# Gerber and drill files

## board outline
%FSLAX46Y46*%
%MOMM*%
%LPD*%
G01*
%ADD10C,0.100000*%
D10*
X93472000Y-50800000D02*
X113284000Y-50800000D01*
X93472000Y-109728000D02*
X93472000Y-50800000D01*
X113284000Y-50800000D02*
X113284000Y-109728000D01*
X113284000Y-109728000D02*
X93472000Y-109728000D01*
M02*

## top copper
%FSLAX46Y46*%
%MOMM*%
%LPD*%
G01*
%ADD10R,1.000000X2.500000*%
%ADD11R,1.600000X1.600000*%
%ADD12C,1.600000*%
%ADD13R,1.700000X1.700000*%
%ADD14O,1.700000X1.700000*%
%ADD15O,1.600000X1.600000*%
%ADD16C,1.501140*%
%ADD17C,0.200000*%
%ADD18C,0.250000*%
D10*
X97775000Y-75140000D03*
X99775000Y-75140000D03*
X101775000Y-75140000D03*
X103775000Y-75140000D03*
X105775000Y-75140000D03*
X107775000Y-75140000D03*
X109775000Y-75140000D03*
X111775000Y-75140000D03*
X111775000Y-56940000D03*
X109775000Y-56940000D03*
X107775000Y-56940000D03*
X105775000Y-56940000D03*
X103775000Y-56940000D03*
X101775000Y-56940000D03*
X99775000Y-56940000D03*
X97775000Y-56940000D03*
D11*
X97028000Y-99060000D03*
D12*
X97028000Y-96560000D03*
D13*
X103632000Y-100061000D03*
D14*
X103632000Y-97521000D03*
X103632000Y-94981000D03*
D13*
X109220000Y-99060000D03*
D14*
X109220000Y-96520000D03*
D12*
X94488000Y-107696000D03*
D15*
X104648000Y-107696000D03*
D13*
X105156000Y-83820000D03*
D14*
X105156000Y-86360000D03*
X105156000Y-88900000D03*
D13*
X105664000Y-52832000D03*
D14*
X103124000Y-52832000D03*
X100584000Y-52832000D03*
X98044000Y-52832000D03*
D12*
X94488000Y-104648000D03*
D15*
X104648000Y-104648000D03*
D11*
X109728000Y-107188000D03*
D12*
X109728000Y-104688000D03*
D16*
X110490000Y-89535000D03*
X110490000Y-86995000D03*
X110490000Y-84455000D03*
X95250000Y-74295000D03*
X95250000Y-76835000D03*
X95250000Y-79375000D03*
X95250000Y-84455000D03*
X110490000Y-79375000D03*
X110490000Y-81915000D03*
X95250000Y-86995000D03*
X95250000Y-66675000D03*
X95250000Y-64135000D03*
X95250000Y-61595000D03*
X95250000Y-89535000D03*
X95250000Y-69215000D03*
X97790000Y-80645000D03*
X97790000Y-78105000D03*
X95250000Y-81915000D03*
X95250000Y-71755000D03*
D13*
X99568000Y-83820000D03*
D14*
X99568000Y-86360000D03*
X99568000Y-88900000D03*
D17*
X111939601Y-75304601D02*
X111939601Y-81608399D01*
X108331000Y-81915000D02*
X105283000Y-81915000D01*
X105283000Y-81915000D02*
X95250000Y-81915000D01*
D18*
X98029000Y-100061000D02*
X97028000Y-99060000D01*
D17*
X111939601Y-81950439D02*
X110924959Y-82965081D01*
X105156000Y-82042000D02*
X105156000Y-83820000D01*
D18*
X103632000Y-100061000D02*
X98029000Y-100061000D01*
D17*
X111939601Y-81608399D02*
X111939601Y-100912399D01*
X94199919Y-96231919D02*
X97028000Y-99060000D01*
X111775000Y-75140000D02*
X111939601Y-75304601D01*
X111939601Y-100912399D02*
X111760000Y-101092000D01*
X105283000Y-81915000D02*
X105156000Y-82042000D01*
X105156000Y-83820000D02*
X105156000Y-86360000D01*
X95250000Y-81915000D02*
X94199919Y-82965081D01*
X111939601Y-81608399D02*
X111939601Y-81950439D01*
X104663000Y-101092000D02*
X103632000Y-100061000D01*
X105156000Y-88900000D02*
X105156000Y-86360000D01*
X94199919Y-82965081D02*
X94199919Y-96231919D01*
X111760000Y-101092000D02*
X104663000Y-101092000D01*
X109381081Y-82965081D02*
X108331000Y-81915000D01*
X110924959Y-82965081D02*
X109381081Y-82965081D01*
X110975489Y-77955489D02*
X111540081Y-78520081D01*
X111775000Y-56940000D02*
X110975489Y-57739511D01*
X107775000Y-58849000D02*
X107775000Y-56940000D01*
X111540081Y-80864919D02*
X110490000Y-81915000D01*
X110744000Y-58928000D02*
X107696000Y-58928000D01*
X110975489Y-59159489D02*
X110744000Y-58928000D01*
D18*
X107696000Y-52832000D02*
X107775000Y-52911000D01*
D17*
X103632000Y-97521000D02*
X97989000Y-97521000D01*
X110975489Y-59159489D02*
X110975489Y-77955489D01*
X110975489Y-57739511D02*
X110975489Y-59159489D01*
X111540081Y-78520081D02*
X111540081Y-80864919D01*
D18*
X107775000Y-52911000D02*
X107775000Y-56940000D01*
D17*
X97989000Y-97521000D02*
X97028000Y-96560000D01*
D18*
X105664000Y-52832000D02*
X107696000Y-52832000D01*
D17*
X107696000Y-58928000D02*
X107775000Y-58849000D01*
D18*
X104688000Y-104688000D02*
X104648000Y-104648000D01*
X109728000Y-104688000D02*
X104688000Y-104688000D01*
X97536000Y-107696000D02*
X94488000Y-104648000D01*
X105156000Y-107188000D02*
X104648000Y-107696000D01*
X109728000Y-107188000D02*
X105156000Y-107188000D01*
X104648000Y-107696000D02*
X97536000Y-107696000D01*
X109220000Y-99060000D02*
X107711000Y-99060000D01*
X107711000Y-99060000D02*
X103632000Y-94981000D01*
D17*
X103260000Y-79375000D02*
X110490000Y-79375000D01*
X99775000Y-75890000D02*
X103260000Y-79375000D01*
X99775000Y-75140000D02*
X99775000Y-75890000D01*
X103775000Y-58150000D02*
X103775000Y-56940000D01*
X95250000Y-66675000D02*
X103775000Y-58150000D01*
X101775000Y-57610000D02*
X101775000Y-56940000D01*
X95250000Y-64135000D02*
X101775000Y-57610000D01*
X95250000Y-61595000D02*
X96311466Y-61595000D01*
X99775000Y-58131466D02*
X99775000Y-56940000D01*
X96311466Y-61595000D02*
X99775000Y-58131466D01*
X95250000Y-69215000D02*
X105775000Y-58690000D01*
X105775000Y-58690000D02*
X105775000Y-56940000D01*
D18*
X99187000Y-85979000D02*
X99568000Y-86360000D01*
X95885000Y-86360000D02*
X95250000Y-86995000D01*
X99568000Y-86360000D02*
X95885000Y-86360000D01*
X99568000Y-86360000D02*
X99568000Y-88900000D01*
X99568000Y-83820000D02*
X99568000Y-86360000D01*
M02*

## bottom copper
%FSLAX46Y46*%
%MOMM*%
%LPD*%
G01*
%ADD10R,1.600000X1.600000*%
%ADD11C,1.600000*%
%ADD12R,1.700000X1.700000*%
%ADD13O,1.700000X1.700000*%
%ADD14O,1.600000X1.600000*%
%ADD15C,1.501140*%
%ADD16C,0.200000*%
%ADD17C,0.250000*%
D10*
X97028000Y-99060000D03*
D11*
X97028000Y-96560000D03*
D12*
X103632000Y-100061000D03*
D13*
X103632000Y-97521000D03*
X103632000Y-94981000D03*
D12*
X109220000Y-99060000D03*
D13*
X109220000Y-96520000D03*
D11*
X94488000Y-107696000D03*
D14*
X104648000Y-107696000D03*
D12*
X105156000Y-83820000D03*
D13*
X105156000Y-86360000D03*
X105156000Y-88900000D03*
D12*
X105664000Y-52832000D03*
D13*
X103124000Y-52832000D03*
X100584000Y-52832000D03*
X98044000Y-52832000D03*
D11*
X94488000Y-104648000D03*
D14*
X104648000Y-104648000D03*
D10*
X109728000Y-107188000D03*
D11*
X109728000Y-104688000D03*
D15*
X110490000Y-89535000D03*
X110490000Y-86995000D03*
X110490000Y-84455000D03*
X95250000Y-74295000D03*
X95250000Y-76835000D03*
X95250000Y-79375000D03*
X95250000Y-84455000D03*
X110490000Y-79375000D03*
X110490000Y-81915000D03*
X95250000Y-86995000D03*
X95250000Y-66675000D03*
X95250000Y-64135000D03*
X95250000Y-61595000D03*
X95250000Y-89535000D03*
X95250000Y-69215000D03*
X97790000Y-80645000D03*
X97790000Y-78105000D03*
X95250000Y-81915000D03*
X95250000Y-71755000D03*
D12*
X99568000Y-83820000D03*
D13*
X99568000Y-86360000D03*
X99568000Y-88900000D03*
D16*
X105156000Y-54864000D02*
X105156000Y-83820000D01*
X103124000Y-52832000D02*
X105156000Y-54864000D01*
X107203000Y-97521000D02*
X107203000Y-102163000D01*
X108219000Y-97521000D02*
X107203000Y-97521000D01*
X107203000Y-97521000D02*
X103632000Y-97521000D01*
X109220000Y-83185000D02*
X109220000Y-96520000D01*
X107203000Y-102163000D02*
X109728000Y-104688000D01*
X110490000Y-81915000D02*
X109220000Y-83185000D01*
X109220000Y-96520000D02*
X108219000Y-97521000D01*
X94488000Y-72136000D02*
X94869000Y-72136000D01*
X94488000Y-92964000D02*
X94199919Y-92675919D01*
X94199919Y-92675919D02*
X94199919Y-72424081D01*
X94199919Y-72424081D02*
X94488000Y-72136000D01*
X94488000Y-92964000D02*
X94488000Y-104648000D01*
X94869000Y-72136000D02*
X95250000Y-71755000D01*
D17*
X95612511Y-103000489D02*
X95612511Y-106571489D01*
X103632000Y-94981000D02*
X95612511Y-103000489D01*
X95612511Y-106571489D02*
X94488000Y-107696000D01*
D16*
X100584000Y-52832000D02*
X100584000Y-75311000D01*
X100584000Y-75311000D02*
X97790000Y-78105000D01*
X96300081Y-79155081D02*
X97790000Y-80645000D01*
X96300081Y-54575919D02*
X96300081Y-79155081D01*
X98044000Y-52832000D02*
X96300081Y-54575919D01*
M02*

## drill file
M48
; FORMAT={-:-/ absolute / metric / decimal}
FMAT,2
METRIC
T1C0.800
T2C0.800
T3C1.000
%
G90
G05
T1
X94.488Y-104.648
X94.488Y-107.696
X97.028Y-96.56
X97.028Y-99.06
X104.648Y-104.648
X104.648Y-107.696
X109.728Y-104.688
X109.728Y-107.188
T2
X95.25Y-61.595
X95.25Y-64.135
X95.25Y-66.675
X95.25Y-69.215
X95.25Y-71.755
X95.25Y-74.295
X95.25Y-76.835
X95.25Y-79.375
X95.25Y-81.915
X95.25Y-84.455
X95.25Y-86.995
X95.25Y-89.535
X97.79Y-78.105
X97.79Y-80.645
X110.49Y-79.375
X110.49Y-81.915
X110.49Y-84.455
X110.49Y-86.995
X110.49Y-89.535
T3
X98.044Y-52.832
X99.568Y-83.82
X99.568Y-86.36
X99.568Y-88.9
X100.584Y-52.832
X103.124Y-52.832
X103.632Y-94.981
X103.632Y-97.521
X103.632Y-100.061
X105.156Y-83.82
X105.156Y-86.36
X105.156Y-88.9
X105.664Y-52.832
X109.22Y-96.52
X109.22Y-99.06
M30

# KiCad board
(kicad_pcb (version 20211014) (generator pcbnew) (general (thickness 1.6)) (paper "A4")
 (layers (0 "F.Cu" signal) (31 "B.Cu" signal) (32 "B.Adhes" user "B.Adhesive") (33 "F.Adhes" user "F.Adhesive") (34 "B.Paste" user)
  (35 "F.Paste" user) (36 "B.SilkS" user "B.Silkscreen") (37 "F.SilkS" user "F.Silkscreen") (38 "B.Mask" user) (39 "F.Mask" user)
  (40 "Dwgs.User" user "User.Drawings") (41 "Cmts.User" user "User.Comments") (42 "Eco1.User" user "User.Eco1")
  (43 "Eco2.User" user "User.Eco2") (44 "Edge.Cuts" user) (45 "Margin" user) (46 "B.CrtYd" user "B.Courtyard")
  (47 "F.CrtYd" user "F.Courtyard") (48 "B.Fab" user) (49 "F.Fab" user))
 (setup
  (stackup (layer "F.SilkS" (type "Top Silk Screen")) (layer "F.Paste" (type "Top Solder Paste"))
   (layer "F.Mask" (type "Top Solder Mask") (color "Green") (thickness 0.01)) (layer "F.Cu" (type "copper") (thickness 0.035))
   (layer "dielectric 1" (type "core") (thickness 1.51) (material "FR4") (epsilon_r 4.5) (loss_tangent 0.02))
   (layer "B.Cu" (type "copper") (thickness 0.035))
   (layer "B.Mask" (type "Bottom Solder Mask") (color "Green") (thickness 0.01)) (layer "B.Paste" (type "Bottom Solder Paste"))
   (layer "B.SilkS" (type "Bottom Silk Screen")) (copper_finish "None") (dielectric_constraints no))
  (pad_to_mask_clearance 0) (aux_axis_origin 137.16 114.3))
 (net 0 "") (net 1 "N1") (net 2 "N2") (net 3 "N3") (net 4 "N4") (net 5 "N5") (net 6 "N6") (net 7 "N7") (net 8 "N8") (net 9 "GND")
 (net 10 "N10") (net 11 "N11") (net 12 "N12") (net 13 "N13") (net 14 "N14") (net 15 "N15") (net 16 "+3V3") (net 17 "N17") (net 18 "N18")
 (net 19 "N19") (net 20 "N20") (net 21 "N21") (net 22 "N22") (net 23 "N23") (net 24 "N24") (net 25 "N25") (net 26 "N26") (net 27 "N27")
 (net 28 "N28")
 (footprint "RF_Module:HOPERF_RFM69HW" (layer "F.Cu") (at 104.775 66.04 90)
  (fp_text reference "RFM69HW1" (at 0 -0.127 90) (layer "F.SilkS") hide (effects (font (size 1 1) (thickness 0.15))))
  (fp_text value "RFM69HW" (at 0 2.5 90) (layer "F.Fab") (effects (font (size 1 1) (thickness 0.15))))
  (pad "1" smd rect (at -9.1 -7 90) (size 2.5 1) (layers "F.Cu" "F.Paste" "F.Mask") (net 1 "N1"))
  (pad "2" smd rect (at -9.1 -5 90) (size 2.5 1) (layers "F.Cu" "F.Paste" "F.Mask") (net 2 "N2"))
  (pad "3" smd rect (at -9.1 -3 90) (size 2.5 1) (layers "F.Cu" "F.Paste" "F.Mask") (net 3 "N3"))
  (pad "4" smd rect (at -9.1 -1 90) (size 2.5 1) (layers "F.Cu" "F.Paste" "F.Mask") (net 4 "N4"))
  (pad "5" smd rect (at -9.1 1 90) (size 2.5 1) (layers "F.Cu" "F.Paste" "F.Mask") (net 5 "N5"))
  (pad "6" smd rect (at -9.1 3 90) (size 2.5 1) (layers "F.Cu" "F.Paste" "F.Mask") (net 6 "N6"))
  (pad "7" smd rect (at -9.1 5 90) (size 2.5 1) (layers "F.Cu" "F.Paste" "F.Mask") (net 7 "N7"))
  (pad "8" smd rect (at -9.1 7 90) (size 2.5 1) (layers "F.Cu" "F.Paste" "F.Mask") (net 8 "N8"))
  (pad "9" smd rect (at 9.1 7 90) (size 2.5 1) (layers "F.Cu" "F.Paste" "F.Mask") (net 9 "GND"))
  (pad "10" smd rect (at 9.1 5 90) (size 2.5 1) (layers "F.Cu" "F.Paste" "F.Mask") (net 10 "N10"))
  (pad "11" smd rect (at 9.1 3 90) (size 2.5 1) (layers "F.Cu" "F.Paste" "F.Mask") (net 9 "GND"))
  (pad "12" smd rect (at 9.1 1 90) (size 2.5 1) (layers "F.Cu" "F.Paste" "F.Mask") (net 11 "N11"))
  (pad "13" smd rect (at 9.1 -1 90) (size 2.5 1) (layers "F.Cu" "F.Paste" "F.Mask") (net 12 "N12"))
  (pad "14" smd rect (at 9.1 -3 90) (size 2.5 1) (layers "F.Cu" "F.Paste" "F.Mask") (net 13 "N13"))
  (pad "15" smd rect (at 9.1 -5 90) (size 2.5 1) (layers "F.Cu" "F.Paste" "F.Mask") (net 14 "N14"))
  (pad "16" smd rect (at 9.1 -7 90) (size 2.5 1) (layers "F.Cu" "F.Paste" "F.Mask") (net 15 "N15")))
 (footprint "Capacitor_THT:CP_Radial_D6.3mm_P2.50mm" (layer "F.Cu") (at 97.028 99.06 90)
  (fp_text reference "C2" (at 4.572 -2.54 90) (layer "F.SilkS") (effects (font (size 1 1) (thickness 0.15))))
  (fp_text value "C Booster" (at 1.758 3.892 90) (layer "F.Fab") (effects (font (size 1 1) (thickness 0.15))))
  (pad "1" thru_hole rect (at 0 0 90) (size 1.6 1.6) (drill 0.8) (layers *.Cu *.Mask) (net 8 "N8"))
  (pad "2" thru_hole circle (at 2.5 0 90) (size 1.6 1.6) (drill 0.8) (layers *.Cu *.Mask) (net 9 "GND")))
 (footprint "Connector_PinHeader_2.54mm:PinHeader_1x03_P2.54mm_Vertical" (layer "F.Cu") (at 103.632 100.061 180)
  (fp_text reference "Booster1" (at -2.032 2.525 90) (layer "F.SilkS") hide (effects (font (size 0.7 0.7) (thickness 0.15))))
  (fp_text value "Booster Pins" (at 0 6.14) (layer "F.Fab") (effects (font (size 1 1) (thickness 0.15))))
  (pad "1" thru_hole rect (at 0 0 180) (size 1.7 1.7) (drill 1) (layers *.Cu *.Mask) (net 8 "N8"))
  (pad "2" thru_hole oval (at 0 2.54 180) (size 1.7 1.7) (drill 1) (layers *.Cu *.Mask) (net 9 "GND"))
  (pad "3" thru_hole oval (at 0 5.08 180) (size 1.7 1.7) (drill 1) (layers *.Cu *.Mask) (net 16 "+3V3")))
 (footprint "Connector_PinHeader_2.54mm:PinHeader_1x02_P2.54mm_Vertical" (layer "F.Cu") (at 109.22 99.06 180)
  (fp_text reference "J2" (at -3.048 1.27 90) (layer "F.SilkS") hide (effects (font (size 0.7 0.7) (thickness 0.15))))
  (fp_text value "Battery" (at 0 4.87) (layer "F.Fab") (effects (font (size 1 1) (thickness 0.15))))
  (pad "1" thru_hole rect (at 0 0 180) (size 1.7 1.7) (drill 1) (layers *.Cu *.Mask) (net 16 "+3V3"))
  (pad "2" thru_hole oval (at 0 2.54 180) (size 1.7 1.7) (drill 1) (layers *.Cu *.Mask) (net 9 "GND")))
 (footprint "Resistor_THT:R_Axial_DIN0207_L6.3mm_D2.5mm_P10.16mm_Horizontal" (layer "F.Cu") (at 94.488 107.696)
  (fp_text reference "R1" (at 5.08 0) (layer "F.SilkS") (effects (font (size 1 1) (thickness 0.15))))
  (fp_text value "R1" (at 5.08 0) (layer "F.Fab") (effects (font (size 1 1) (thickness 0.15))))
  (pad "1" thru_hole circle (at 0 0) (size 1.6 1.6) (drill 0.8) (layers *.Cu *.Mask) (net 16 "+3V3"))
  (pad "2" thru_hole oval (at 10.16 0) (size 1.6 1.6) (drill 0.8) (layers *.Cu *.Mask) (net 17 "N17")))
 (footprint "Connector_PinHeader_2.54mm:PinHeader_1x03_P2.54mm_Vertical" (layer "F.Cu") (at 105.156 83.82)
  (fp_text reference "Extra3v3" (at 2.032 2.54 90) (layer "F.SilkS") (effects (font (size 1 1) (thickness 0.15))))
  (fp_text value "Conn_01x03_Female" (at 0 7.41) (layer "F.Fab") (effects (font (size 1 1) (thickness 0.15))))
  (pad "1" thru_hole rect (at 0 0) (size 1.7 1.7) (drill 1) (layers *.Cu *.Mask) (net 8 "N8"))
  (pad "2" thru_hole oval (at 0 2.54) (size 1.7 1.7) (drill 1) (layers *.Cu *.Mask) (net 8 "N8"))
  (pad "3" thru_hole oval (at 0 5.08) (size 1.7 1.7) (drill 1) (layers *.Cu *.Mask) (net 8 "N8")))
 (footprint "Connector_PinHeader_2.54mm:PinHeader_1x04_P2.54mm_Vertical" (layer "F.Cu") (at 105.664 52.832 -90)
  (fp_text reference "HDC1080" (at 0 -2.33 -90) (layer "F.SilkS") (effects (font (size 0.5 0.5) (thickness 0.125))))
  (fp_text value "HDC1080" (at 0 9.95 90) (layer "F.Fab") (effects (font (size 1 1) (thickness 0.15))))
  (pad "1" thru_hole rect (at 0 0 270) (size 1.7 1.7) (drill 1) (layers *.Cu *.Mask) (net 9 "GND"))
  (pad "2" thru_hole oval (at 0 2.54 270) (size 1.7 1.7) (drill 1) (layers *.Cu *.Mask) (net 8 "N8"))
  (pad "3" thru_hole oval (at 0 5.08 270) (size 1.7 1.7) (drill 1) (layers *.Cu *.Mask) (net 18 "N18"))
  (pad "4" thru_hole oval (at 0 7.62 270) (size 1.7 1.7) (drill 1) (layers *.Cu *.Mask) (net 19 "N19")))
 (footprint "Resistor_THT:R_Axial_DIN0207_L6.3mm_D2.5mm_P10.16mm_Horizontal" (layer "F.Cu") (at 94.488 104.648)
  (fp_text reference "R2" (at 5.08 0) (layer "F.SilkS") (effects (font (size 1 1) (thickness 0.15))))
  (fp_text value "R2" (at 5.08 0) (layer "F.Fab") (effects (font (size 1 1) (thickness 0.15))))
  (pad "1" thru_hole circle (at 0 0) (size 1.6 1.6) (drill 0.8) (layers *.Cu *.Mask) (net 17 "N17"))
  (pad "2" thru_hole oval (at 10.16 0) (size 1.6 1.6) (drill 0.8) (layers *.Cu *.Mask) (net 9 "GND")))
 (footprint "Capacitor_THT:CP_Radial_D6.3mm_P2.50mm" (layer "F.Cu") (at 109.728 107.188 90)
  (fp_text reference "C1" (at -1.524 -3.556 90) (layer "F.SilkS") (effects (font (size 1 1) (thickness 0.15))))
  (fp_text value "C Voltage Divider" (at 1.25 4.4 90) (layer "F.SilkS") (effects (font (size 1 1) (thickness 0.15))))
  (pad "1" thru_hole rect (at 0 0 90) (size 1.6 1.6) (drill 0.8) (layers *.Cu *.Mask) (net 17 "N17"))
  (pad "2" thru_hole circle (at 2.5 0 90) (size 1.6 1.6) (drill 0.8) (layers *.Cu *.Mask) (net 9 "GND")))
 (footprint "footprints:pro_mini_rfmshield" (layer "F.Cu") (at 102.87 75.565)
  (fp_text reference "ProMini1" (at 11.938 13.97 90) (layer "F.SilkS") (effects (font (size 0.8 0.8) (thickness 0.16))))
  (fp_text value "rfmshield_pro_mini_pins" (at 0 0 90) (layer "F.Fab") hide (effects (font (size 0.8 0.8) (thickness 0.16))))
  (pad "1" thru_hole circle (at 7.62 13.97 90) (size 1.50114 1.50114) (drill 0.8001) (layers *.Cu *.Mask "F.SilkS") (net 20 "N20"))
  (pad "2" thru_hole circle (at 7.62 11.43 90) (size 1.50114 1.50114) (drill 0.8001) (layers *.Cu *.Mask "F.SilkS") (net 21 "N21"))
  (pad "3" thru_hole circle (at 7.62 8.89 90) (size 1.50114 1.50114) (drill 0.8001) (layers *.Cu *.Mask "F.SilkS") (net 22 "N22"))
  (pad "18" thru_hole circle (at -7.62 -1.27 90) (size 1.50114 1.50114) (drill 0.8001) (layers *.Cu *.Mask "F.SilkS") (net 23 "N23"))
  (pad "19" thru_hole circle (at -7.62 1.27 90) (size 1.50114 1.50114) (drill 0.8001) (layers *.Cu *.Mask "F.SilkS") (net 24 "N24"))
  (pad "20" thru_hole circle (at -7.62 3.81 90) (size 1.50114 1.50114) (drill 0.8001) (layers *.Cu *.Mask "F.SilkS") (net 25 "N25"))
  (pad "22" thru_hole circle (at -7.62 8.89 90) (size 1.50114 1.50114) (drill 0.8001) (layers *.Cu *.Mask "F.SilkS") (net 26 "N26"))
  (pad "DI00" thru_hole circle (at 7.62 3.81 90) (size 1.50114 1.50114) (drill 0.8001) (layers *.Cu *.Mask "F.SilkS") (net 2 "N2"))
  (pad "GND1" thru_hole circle (at 7.62 6.35 90) (size 1.50114 1.50114) (drill 0.8001) (layers *.Cu *.Mask "F.SilkS") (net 9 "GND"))
  (pad "GND2" thru_hole circle (at -7.62 11.43 90) (size 1.50114 1.50114) (drill 0.8001) (layers *.Cu *.Mask "F.SilkS") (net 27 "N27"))
  (pad "MISO" thru_hole circle (at -7.62 -8.89 90) (size 1.50114 1.50114) (drill 0.8001) (layers *.Cu *.Mask "F.SilkS") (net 12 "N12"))
  (pad "MOSI" thru_hole circle (at -7.62 -11.43 90) (size 1.50114 1.50114) (drill 0.8001) (layers *.Cu *.Mask "F.SilkS") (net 13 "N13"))
  (pad "NSS" thru_hole circle (at -7.62 -13.97 90) (size 1.50114 1.50114) (drill 0.8001) (layers *.Cu *.Mask "F.SilkS") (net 14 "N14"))
  (pad "RAW" thru_hole circle (at -7.62 13.97 90) (size 1.50114 1.50114) (drill 0.8001) (layers *.Cu *.Mask "F.SilkS") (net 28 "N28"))
  (pad "SCK" thru_hole circle (at -7.62 -6.35 90) (size 1.50114 1.50114) (drill 0.8001) (layers *.Cu *.Mask "F.SilkS") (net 11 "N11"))
  (pad "SCL" thru_hole circle (at -5.08 5.08 90) (size 1.50114 1.50114) (drill 0.8001) (layers *.Cu *.Mask "F.SilkS") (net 19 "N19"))
  (pad "SDA" thru_hole circle (at -5.08 2.54 90) (size 1.50114 1.50114) (drill 0.8001) (layers *.Cu *.Mask "F.SilkS") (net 18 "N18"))
  (pad "VCC" thru_hole circle (at -7.62 6.35 90) (size 1.50114 1.50114) (drill 0.8001) (layers *.Cu *.Mask "F.SilkS") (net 8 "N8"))
  (pad "VolDiv" thru_hole circle (at -7.62 -3.81 90) (size 1.50114 1.50114) (drill 0.8001) (layers *.Cu *.Mask "F.SilkS") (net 17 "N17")))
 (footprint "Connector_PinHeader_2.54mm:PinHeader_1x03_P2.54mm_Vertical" (layer "F.Cu") (at 99.568 83.82)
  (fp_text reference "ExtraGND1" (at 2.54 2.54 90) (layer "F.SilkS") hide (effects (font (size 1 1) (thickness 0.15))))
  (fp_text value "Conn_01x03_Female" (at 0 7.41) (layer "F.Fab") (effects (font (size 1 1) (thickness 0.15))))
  (pad "1" thru_hole rect (at 0 0) (size 1.7 1.7) (drill 1) (layers *.Cu *.Mask) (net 27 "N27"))
  (pad "2" thru_hole oval (at 0 2.54) (size 1.7 1.7) (drill 1) (layers *.Cu *.Mask) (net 27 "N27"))
  (pad "3" thru_hole oval (at 0 5.08) (size 1.7 1.7) (drill 1) (layers *.Cu *.Mask) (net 27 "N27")))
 (gr_line (start 93.472 50.8) (end 113.284 50.8) (layer "Edge.Cuts") (width 0.1))
 (gr_line (start 93.472 109.728) (end 93.472 50.8) (layer "Edge.Cuts") (width 0.1))
 (gr_line (start 113.284 50.8) (end 113.284 109.728) (layer "Edge.Cuts") (width 0.1))
 (gr_line (start 113.284 109.728) (end 93.472 109.728) (layer "Edge.Cuts") (width 0.1))
 (segment (start 111.939601 75.304601) (end 111.939601 81.608399) (width 0.2) (layer "F.Cu") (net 8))
 (segment (start 108.331 81.915) (end 105.283 81.915) (width 0.2) (layer "F.Cu") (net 8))
 (segment (start 105.283 81.915) (end 95.25 81.915) (width 0.2) (layer "F.Cu") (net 8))
 (segment (start 98.029 100.061) (end 97.028 99.06) (width 0.25) (layer "F.Cu") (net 8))
 (segment (start 111.939601 81.950439) (end 110.924959 82.965081) (width 0.2) (layer "F.Cu") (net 8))
 (segment (start 105.156 82.042) (end 105.156 83.82) (width 0.2) (layer "F.Cu") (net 8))
 (segment (start 103.632 100.061) (end 98.029 100.061) (width 0.25) (layer "F.Cu") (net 8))
 (segment (start 111.939601 81.608399) (end 111.939601 100.912399) (width 0.2) (layer "F.Cu") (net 8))
 (segment (start 94.199919 96.231919) (end 97.028 99.06) (width 0.2) (layer "F.Cu") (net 8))
 (segment (start 111.775 75.14) (end 111.939601 75.304601) (width 0.2) (layer "F.Cu") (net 8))
 (segment (start 111.939601 100.912399) (end 111.76 101.092) (width 0.2) (layer "F.Cu") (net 8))
 (segment (start 105.283 81.915) (end 105.156 82.042) (width 0.2) (layer "F.Cu") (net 8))
 (segment (start 105.156 83.82) (end 105.156 86.36) (width 0.2) (layer "F.Cu") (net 8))
 (segment (start 95.25 81.915) (end 94.199919 82.965081) (width 0.2) (layer "F.Cu") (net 8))
 (segment (start 111.939601 81.608399) (end 111.939601 81.950439) (width 0.2) (layer "F.Cu") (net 8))
 (segment (start 104.663 101.092) (end 103.632 100.061) (width 0.2) (layer "F.Cu") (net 8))
 (segment (start 105.156 88.9) (end 105.156 86.36) (width 0.2) (layer "F.Cu") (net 8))
 (segment (start 94.199919 82.965081) (end 94.199919 96.231919) (width 0.2) (layer "F.Cu") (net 8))
 (segment (start 111.76 101.092) (end 104.663 101.092) (width 0.2) (layer "F.Cu") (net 8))
 (segment (start 109.381081 82.965081) (end 108.331 81.915) (width 0.2) (layer "F.Cu") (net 8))
 (segment (start 110.924959 82.965081) (end 109.381081 82.965081) (width 0.2) (layer "F.Cu") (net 8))
 (segment (start 105.156 54.864) (end 105.156 83.82) (width 0.2) (layer "B.Cu") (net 8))
 (segment (start 103.124 52.832) (end 105.156 54.864) (width 0.2) (layer "B.Cu") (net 8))
 (segment (start 110.975489 77.955489) (end 111.540081 78.520081) (width 0.2) (layer "F.Cu") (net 9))
 (segment (start 111.775 56.94) (end 110.975489 57.739511) (width 0.2) (layer "F.Cu") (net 9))
 (segment (start 107.775 58.849) (end 107.775 56.94) (width 0.2) (layer "F.Cu") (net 9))
 (segment (start 111.540081 80.864919) (end 110.49 81.915) (width 0.2) (layer "F.Cu") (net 9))
 (segment (start 110.744 58.928) (end 107.696 58.928) (width 0.2) (layer "F.Cu") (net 9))
 (segment (start 110.975489 59.159489) (end 110.744 58.928) (width 0.2) (layer "F.Cu") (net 9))
 (segment (start 107.696 52.832) (end 107.775 52.911) (width 0.25) (layer "F.Cu") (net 9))
 (segment (start 103.632 97.521) (end 97.989 97.521) (width 0.2) (layer "F.Cu") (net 9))
 (segment (start 110.975489 59.159489) (end 110.975489 77.955489) (width 0.2) (layer "F.Cu") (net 9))
 (segment (start 110.975489 57.739511) (end 110.975489 59.159489) (width 0.2) (layer "F.Cu") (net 9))
 (segment (start 111.540081 78.520081) (end 111.540081 80.864919) (width 0.2) (layer "F.Cu") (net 9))
 (segment (start 107.775 52.911) (end 107.775 56.94) (width 0.25) (layer "F.Cu") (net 9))
 (segment (start 97.989 97.521) (end 97.028 96.56) (width 0.2) (layer "F.Cu") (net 9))
 (segment (start 105.664 52.832) (end 107.696 52.832) (width 0.25) (layer "F.Cu") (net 9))
 (segment (start 107.696 58.928) (end 107.775 58.849) (width 0.2) (layer "F.Cu") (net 9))
 (segment (start 104.688 104.688) (end 104.648 104.648) (width 0.25) (layer "F.Cu") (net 9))
 (segment (start 109.728 104.688) (end 104.688 104.688) (width 0.25) (layer "F.Cu") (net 9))
 (segment (start 107.203 97.521) (end 107.203 102.163) (width 0.2) (layer "B.Cu") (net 9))
 (segment (start 108.219 97.521) (end 107.203 97.521) (width 0.2) (layer "B.Cu") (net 9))
 (segment (start 107.203 97.521) (end 103.632 97.521) (width 0.2) (layer "B.Cu") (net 9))
 (segment (start 109.22 83.185) (end 109.22 96.52) (width 0.2) (layer "B.Cu") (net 9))
 (segment (start 107.203 102.163) (end 109.728 104.688) (width 0.2) (layer "B.Cu") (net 9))
 (segment (start 110.49 81.915) (end 109.22 83.185) (width 0.2) (layer "B.Cu") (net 9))
 (segment (start 109.22 96.52) (end 108.219 97.521) (width 0.2) (layer "B.Cu") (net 9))
 (segment (start 97.536 107.696) (end 94.488 104.648) (width 0.25) (layer "F.Cu") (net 17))
 (segment (start 105.156 107.188) (end 104.648 107.696) (width 0.25) (layer "F.Cu") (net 17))
 (segment (start 109.728 107.188) (end 105.156 107.188) (width 0.25) (layer "F.Cu") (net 17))
 (segment (start 104.648 107.696) (end 97.536 107.696) (width 0.25) (layer "F.Cu") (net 17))
 (segment (start 94.488 72.136) (end 94.869 72.136) (width 0.2) (layer "B.Cu") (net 17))
 (segment (start 94.488 92.964) (end 94.199919 92.675919) (width 0.2) (layer "B.Cu") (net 17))
 (segment (start 94.199919 92.675919) (end 94.199919 72.424081) (width 0.2) (layer "B.Cu") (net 17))
 (segment (start 94.199919 72.424081) (end 94.488 72.136) (width 0.2) (layer "B.Cu") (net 17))
 (segment (start 94.488 92.964) (end 94.488 104.648) (width 0.2) (layer "B.Cu") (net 17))
 (segment (start 94.869 72.136) (end 95.25 71.755) (width 0.2) (layer "B.Cu") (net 17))
 (segment (start 109.22 99.06) (end 107.711 99.06) (width 0.25) (layer "F.Cu") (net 16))
 (segment (start 107.711 99.06) (end 103.632 94.981) (width 0.25) (layer "F.Cu") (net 16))
 (segment (start 95.612511 103.000489) (end 95.612511 106.571489) (width 0.25) (layer "B.Cu") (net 16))
 (segment (start 103.632 94.981) (end 95.612511 103.000489) (width 0.25) (layer "B.Cu") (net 16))
 (segment (start 95.612511 106.571489) (end 94.488 107.696) (width 0.25) (layer "B.Cu") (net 16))
 (segment (start 103.26 79.375) (end 110.49 79.375) (width 0.2) (layer "F.Cu") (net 2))
 (segment (start 99.775 75.89) (end 103.26 79.375) (width 0.2) (layer "F.Cu") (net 2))
 (segment (start 99.775 75.14) (end 99.775 75.89) (width 0.2) (layer "F.Cu") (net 2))
 (segment (start 103.775 58.15) (end 103.775 56.94) (width 0.2) (layer "F.Cu") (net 12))
 (segment (start 95.25 66.675) (end 103.775 58.15) (width 0.2) (layer "F.Cu") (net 12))
 (segment (start 101.775 57.61) (end 101.775 56.94) (width 0.2) (layer "F.Cu") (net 13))
 (segment (start 95.25 64.135) (end 101.775 57.61) (width 0.2) (layer "F.Cu") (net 13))
 (segment (start 95.25 61.595) (end 96.311466 61.595) (width 0.2) (layer "F.Cu") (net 14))
 (segment (start 99.775 58.131466) (end 99.775 56.94) (width 0.2) (layer "F.Cu") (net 14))
 (segment (start 96.311466 61.595) (end 99.775 58.131466) (width 0.2) (layer "F.Cu") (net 14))
 (segment (start 95.25 69.215) (end 105.775 58.69) (width 0.2) (layer "F.Cu") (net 11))
 (segment (start 105.775 58.69) (end 105.775 56.94) (width 0.2) (layer "F.Cu") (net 11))
 (segment (start 100.584 52.832) (end 100.584 75.311) (width 0.2) (layer "B.Cu") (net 18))
 (segment (start 100.584 75.311) (end 97.79 78.105) (width 0.2) (layer "B.Cu") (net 18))
 (segment (start 96.300081 79.155081) (end 97.79 80.645) (width 0.2) (layer "B.Cu") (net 19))
 (segment (start 96.300081 54.575919) (end 96.300081 79.155081) (width 0.2) (layer "B.Cu") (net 19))
 (segment (start 98.044 52.832) (end 96.300081 54.575919) (width 0.2) (layer "B.Cu") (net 19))
 (segment (start 99.187 85.979) (end 99.568 86.36) (width 0.25) (layer "F.Cu") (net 27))
 (segment (start 95.885 86.36) (end 95.25 86.995) (width 0.25) (layer "F.Cu") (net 27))
 (segment (start 99.568 86.36) (end 95.885 86.36) (width 0.25) (layer "F.Cu") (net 27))
 (segment (start 99.568 86.36) (end 99.568 88.9) (width 0.25) (layer "F.Cu") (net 27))
 (segment (start 99.568 83.82) (end 99.568 86.36) (width 0.25) (layer "F.Cu") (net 27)))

